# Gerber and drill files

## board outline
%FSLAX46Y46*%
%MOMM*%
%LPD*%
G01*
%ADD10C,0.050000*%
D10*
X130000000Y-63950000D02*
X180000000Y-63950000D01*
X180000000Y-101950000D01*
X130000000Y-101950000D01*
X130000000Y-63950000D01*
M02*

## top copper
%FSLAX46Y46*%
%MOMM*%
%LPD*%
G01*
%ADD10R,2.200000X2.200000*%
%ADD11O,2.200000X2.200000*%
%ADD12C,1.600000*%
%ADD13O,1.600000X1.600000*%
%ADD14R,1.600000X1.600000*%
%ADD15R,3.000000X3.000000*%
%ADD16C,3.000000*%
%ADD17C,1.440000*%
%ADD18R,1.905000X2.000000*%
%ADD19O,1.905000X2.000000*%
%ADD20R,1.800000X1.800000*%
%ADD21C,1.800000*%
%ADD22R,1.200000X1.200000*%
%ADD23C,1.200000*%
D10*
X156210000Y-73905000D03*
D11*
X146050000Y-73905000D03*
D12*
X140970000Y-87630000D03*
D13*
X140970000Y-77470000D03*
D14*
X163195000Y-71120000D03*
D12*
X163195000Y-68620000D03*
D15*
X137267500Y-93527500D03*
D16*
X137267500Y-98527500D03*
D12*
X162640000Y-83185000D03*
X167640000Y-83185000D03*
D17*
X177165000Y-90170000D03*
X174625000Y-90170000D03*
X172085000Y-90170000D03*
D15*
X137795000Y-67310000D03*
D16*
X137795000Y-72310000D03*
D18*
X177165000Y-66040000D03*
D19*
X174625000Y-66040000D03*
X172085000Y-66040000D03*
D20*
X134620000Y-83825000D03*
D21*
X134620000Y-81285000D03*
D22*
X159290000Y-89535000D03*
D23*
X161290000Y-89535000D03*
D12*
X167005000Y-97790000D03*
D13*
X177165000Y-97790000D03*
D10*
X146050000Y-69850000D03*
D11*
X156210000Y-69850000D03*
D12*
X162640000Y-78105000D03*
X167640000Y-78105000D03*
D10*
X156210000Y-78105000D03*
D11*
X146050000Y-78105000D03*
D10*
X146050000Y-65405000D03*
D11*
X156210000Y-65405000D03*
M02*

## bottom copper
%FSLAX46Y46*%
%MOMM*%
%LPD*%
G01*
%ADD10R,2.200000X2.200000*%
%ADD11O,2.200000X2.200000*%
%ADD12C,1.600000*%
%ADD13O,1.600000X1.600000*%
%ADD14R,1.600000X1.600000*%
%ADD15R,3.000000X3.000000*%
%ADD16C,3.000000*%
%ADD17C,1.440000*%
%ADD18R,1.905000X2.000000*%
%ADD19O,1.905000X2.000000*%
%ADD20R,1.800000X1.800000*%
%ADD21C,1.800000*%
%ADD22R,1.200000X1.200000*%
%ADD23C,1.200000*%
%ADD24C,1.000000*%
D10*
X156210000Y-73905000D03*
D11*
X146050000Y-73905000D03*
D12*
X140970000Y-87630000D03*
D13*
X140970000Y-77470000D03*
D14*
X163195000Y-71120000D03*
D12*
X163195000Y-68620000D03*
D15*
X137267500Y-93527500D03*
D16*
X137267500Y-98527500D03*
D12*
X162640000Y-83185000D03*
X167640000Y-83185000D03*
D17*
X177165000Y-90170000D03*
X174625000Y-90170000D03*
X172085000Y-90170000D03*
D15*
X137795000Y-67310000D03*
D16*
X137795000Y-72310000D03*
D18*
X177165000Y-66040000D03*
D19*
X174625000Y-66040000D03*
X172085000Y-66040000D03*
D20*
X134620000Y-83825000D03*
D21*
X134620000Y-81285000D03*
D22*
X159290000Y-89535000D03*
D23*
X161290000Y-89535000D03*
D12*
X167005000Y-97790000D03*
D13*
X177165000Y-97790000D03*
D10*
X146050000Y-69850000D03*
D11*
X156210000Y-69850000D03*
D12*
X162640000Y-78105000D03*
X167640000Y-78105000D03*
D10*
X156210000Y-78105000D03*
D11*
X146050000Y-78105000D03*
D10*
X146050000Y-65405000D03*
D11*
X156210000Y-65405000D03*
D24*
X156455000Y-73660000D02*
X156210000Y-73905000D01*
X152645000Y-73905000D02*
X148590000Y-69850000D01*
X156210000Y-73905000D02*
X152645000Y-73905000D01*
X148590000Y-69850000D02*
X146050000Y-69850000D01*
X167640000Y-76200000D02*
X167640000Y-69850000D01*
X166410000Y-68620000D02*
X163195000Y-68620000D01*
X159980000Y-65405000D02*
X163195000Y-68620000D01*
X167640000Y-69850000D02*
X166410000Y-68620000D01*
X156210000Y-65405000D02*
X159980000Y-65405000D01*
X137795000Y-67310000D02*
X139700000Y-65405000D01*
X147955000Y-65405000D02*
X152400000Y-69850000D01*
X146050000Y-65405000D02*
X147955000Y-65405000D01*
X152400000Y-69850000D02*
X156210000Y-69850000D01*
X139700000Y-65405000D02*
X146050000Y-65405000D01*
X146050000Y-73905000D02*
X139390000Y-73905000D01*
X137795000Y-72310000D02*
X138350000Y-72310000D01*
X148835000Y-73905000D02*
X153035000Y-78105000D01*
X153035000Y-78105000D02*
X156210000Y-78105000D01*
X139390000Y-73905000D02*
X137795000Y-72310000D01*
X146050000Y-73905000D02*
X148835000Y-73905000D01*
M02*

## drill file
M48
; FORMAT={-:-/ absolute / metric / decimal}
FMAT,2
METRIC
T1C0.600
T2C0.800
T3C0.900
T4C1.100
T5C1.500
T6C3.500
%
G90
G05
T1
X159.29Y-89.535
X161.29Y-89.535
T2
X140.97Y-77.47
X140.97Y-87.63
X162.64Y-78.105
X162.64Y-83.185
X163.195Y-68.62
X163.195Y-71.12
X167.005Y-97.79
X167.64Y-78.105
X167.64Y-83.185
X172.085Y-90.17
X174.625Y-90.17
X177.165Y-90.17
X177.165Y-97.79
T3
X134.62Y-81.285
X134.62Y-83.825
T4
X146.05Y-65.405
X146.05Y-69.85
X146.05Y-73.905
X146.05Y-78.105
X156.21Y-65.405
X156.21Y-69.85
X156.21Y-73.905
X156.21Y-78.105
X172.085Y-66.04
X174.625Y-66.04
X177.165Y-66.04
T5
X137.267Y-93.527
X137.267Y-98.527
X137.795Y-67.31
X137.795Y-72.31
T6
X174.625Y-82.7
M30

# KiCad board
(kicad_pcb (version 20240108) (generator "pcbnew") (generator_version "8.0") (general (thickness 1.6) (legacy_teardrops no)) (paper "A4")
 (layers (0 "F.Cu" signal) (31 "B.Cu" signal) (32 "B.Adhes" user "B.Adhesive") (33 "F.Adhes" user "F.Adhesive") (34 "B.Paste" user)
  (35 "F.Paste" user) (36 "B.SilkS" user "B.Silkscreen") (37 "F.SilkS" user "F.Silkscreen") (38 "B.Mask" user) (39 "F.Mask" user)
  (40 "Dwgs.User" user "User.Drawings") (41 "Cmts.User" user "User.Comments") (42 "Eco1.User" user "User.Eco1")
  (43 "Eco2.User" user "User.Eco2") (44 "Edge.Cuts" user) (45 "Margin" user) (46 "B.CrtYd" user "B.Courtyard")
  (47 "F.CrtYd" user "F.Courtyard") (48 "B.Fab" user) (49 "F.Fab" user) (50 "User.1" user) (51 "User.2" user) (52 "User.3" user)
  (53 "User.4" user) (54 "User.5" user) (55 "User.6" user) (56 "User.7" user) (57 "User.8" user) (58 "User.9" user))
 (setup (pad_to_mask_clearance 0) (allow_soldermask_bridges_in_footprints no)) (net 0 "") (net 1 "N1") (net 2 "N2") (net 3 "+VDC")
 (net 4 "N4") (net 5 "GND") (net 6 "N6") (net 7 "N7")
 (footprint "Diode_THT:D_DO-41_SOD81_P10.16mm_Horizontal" (layer "F.Cu") (at 156.21 73.905 180)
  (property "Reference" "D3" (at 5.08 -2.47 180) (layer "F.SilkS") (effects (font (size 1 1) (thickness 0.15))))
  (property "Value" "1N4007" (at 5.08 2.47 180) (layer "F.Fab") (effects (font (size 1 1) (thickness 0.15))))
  (pad "1" thru_hole rect (at 0 0 180) (size 2.2 2.2) (drill 1.1) (layers "*.Cu" "*.Mask") (remove_unused_layers no) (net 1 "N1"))
  (pad "2" thru_hole oval (at 10.16 0 180) (size 2.2 2.2) (drill 1.1) (layers "*.Cu" "*.Mask") (remove_unused_layers no) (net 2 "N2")))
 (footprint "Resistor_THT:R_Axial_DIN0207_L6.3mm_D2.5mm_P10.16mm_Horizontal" (layer "F.Cu") (at 140.97 87.63 90)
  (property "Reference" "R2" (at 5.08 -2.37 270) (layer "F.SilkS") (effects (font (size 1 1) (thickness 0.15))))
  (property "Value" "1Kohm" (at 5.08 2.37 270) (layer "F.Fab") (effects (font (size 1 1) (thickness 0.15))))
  (pad "1" thru_hole circle (at 0 0 90) (size 1.6 1.6) (drill 0.8) (layers "*.Cu" "*.Mask") (remove_unused_layers no) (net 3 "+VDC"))
  (pad "2" thru_hole oval (at 10.16 0 90) (size 1.6 1.6) (drill 0.8) (layers "*.Cu" "*.Mask") (remove_unused_layers no) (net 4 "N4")))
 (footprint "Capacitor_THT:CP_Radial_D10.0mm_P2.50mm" (layer "F.Cu") (at 163.195 71.12 90)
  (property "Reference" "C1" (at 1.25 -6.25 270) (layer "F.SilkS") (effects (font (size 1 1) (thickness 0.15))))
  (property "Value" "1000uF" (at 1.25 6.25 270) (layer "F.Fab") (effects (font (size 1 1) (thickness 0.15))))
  (pad "1" thru_hole rect (at 0 0 90) (size 1.6 1.6) (drill 0.8) (layers "*.Cu" "*.Mask") (remove_unused_layers no) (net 1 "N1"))
  (pad "2" thru_hole circle (at 2.5 0 90) (size 1.6 1.6) (drill 0.8) (layers "*.Cu" "*.Mask") (remove_unused_layers no) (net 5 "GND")))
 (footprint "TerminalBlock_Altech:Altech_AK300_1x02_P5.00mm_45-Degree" (layer "F.Cu") (at 137.2675 93.5275 -90)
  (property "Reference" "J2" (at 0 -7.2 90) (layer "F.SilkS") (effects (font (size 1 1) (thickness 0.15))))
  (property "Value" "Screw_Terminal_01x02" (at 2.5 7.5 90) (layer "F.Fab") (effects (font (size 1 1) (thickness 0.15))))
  (pad "1" thru_hole rect (at 0 0 270) (size 3 3) (drill 1.5) (layers "*.Cu" "*.Mask") (remove_unused_layers no) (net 3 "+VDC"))
  (pad "2" thru_hole circle (at 5 0 270) (size 3 3) (drill 1.5) (layers "*.Cu" "*.Mask") (remove_unused_layers no) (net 5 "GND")))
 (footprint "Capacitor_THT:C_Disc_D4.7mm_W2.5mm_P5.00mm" (layer "F.Cu") (at 162.64 83.185)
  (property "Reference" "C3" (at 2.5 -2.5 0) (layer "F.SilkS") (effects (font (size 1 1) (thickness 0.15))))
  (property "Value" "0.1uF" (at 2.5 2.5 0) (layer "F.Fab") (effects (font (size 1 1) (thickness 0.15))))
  (pad "1" thru_hole circle (at 0 0) (size 1.6 1.6) (drill 0.8) (layers "*.Cu" "*.Mask") (remove_unused_layers no) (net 3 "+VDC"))
  (pad "2" thru_hole circle (at 5 0) (size 1.6 1.6) (drill 0.8) (layers "*.Cu" "*.Mask") (remove_unused_layers no) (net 5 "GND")))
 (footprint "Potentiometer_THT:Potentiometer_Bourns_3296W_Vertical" (layer "F.Cu") (at 177.165 90.17)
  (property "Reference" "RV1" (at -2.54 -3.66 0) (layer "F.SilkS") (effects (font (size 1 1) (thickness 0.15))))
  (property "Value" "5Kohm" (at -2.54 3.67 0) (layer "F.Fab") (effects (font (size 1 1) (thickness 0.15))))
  (pad "1" thru_hole circle (at 0 0) (size 1.44 1.44) (drill 0.8) (layers "*.Cu" "*.Mask") (remove_unused_layers no) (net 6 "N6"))
  (pad "2" thru_hole circle (at -2.54 0) (size 1.44 1.44) (drill 0.8) (layers "*.Cu" "*.Mask") (remove_unused_layers no) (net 5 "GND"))
  (pad "3" thru_hole circle (at -5.08 0) (size 1.44 1.44) (drill 0.8) (layers "*.Cu" "*.Mask") (remove_unused_layers no) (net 5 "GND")))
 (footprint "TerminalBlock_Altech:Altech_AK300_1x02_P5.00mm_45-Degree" (layer "F.Cu") (at 137.795 67.31 -90)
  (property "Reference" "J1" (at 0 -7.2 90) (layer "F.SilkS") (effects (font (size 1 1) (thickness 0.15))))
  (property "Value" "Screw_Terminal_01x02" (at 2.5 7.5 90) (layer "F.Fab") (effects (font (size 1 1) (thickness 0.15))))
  (pad "1" thru_hole rect (at 0 0 270) (size 3 3) (drill 1.5) (layers "*.Cu" "*.Mask") (remove_unused_layers no) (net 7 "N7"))
  (pad "2" thru_hole circle (at 5 0 270) (size 3 3) (drill 1.5) (layers "*.Cu" "*.Mask") (remove_unused_layers no) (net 2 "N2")))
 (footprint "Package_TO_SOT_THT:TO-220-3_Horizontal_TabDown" (layer "F.Cu") (at 177.165 66.04 180)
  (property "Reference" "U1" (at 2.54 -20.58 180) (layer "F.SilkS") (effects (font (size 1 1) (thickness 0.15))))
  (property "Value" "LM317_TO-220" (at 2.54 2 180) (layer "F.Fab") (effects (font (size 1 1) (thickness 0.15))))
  (pad "" np_thru_hole oval (at 2.54 -16.66 180) (size 3.5 3.5) (drill 3.5) (layers "*.Cu" "*.Mask"))
  (pad "1" thru_hole rect (at 0 0 180) (size 1.905 2) (drill 1.1) (layers "*.Cu" "*.Mask") (remove_unused_layers no) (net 6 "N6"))
  (pad "2" thru_hole oval (at 2.54 0 180) (size 1.905 2) (drill 1.1) (layers "*.Cu" "*.Mask") (remove_unused_layers no) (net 3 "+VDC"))
  (pad "3" thru_hole oval (at 5.08 0 180) (size 1.905 2) (drill 1.1) (layers "*.Cu" "*.Mask") (remove_unused_layers no) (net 1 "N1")))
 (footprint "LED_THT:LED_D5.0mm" (layer "F.Cu") (at 134.62 83.825 90)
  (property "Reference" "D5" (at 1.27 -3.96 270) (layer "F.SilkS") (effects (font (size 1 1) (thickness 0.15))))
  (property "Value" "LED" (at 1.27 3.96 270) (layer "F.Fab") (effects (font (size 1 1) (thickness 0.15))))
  (pad "1" thru_hole rect (at 0 0 90) (size 1.8 1.8) (drill 0.9) (layers "*.Cu" "*.Mask") (remove_unused_layers no) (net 5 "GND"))
  (pad "2" thru_hole circle (at 2.54 0 90) (size 1.8 1.8) (drill 0.9) (layers "*.Cu" "*.Mask") (remove_unused_layers no) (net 4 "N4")))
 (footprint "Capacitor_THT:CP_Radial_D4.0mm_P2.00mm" (layer "F.Cu") (at 159.29 89.535)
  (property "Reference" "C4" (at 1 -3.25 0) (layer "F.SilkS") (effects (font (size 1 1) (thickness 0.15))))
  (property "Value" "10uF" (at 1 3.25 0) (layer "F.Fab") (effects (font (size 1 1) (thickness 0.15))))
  (pad "1" thru_hole rect (at 0 0) (size 1.2 1.2) (drill 0.6) (layers "*.Cu" "*.Mask") (remove_unused_layers no) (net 3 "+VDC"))
  (pad "2" thru_hole circle (at 2 0) (size 1.2 1.2) (drill 0.6) (layers "*.Cu" "*.Mask") (remove_unused_layers no) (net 5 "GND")))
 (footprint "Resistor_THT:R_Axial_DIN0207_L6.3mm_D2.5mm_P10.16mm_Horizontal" (layer "F.Cu") (at 167.005 97.79)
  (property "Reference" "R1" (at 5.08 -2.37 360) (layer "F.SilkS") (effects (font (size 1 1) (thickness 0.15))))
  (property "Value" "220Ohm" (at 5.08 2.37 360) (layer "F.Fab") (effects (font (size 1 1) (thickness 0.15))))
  (pad "1" thru_hole circle (at 0 0) (size 1.6 1.6) (drill 0.8) (layers "*.Cu" "*.Mask") (remove_unused_layers no) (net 3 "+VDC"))
  (pad "2" thru_hole oval (at 10.16 0) (size 1.6 1.6) (drill 0.8) (layers "*.Cu" "*.Mask") (remove_unused_layers no) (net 6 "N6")))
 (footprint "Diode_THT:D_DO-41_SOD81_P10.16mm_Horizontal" (layer "F.Cu") (at 146.05 69.85)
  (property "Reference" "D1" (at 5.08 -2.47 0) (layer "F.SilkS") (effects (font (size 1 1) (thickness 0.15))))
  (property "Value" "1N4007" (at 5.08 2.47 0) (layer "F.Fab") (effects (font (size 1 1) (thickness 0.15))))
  (pad "1" thru_hole rect (at 0 0) (size 2.2 2.2) (drill 1.1) (layers "*.Cu" "*.Mask") (remove_unused_layers no) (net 1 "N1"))
  (pad "2" thru_hole oval (at 10.16 0) (size 2.2 2.2) (drill 1.1) (layers "*.Cu" "*.Mask") (remove_unused_layers no) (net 7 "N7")))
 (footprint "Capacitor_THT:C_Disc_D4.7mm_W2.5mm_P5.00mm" (layer "F.Cu") (at 162.64 78.105)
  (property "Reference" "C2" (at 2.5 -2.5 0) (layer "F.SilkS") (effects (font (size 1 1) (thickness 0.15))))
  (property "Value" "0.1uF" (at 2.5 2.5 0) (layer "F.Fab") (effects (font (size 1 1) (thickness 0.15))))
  (pad "1" thru_hole circle (at 0 0) (size 1.6 1.6) (drill 0.8) (layers "*.Cu" "*.Mask") (remove_unused_layers no) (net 1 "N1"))
  (pad "2" thru_hole circle (at 5 0) (size 1.6 1.6) (drill 0.8) (layers "*.Cu" "*.Mask") (remove_unused_layers no) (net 5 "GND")))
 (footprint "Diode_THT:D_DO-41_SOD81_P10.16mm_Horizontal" (layer "F.Cu") (at 156.21 78.105 180)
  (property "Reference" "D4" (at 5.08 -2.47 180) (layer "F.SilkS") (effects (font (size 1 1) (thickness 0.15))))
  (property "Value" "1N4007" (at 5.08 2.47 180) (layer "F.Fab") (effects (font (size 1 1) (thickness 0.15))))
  (pad "1" thru_hole rect (at 0 0 180) (size 2.2 2.2) (drill 1.1) (layers "*.Cu" "*.Mask") (remove_unused_layers no) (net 2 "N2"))
  (pad "2" thru_hole oval (at 10.16 0 180) (size 2.2 2.2) (drill 1.1) (layers "*.Cu" "*.Mask") (remove_unused_layers no) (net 5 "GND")))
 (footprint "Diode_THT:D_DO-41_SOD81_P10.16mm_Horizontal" (layer "F.Cu") (at 146.05 65.405)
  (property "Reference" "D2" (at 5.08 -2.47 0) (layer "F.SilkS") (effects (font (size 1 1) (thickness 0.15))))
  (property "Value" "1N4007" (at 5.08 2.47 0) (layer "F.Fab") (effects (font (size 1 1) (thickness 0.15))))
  (pad "1" thru_hole rect (at 0 0) (size 2.2 2.2) (drill 1.1) (layers "*.Cu" "*.Mask") (remove_unused_layers no) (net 7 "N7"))
  (pad "2" thru_hole oval (at 10.16 0) (size 2.2 2.2) (drill 1.1) (layers "*.Cu" "*.Mask") (remove_unused_layers no) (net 5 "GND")))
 (gr_rect (start 130 63.95) (end 180 101.95) (stroke (width 0.05) (type default)) (fill none) (layer "Edge.Cuts"))
 (segment (start 156.455 73.66) (end 156.21 73.905) (width 1) (layer "B.Cu") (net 1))
 (segment (start 152.645 73.905) (end 148.59 69.85) (width 1) (layer "B.Cu") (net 1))
 (segment (start 156.21 73.905) (end 152.645 73.905) (width 1) (layer "B.Cu") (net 1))
 (segment (start 148.59 69.85) (end 146.05 69.85) (width 1) (layer "B.Cu") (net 1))
 (segment (start 167.64 76.2) (end 167.64 69.85) (width 1) (layer "B.Cu") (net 5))
 (segment (start 166.41 68.62) (end 163.195 68.62) (width 1) (layer "B.Cu") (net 5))
 (segment (start 159.98 65.405) (end 163.195 68.62) (width 1) (layer "B.Cu") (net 5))
 (segment (start 167.64 69.85) (end 166.41 68.62) (width 1) (layer "B.Cu") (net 5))
 (segment (start 156.21 65.405) (end 159.98 65.405) (width 1) (layer "B.Cu") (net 5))
 (segment (start 137.795 67.31) (end 139.7 65.405) (width 1) (layer "B.Cu") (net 7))
 (segment (start 147.955 65.405) (end 152.4 69.85) (width 1) (layer "B.Cu") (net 7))
 (segment (start 146.05 65.405) (end 147.955 65.405) (width 1) (layer "B.Cu") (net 7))
 (segment (start 152.4 69.85) (end 156.21 69.85) (width 1) (layer "B.Cu") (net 7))
 (segment (start 139.7 65.405) (end 146.05 65.405) (width 1) (layer "B.Cu") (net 7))
 (segment (start 146.05 73.905) (end 139.39 73.905) (width 1) (layer "B.Cu") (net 2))
 (segment (start 137.795 72.31) (end 138.35 72.31) (width 1) (layer "B.Cu") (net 2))
 (segment (start 148.835 73.905) (end 153.035 78.105) (width 1) (layer "B.Cu") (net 2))
 (segment (start 153.035 78.105) (end 156.21 78.105) (width 1) (layer "B.Cu") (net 2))
 (segment (start 139.39 73.905) (end 137.795 72.31) (width 1) (layer "B.Cu") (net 2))
 (segment (start 146.05 73.905) (end 148.835 73.905) (width 1) (layer "B.Cu") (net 2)))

